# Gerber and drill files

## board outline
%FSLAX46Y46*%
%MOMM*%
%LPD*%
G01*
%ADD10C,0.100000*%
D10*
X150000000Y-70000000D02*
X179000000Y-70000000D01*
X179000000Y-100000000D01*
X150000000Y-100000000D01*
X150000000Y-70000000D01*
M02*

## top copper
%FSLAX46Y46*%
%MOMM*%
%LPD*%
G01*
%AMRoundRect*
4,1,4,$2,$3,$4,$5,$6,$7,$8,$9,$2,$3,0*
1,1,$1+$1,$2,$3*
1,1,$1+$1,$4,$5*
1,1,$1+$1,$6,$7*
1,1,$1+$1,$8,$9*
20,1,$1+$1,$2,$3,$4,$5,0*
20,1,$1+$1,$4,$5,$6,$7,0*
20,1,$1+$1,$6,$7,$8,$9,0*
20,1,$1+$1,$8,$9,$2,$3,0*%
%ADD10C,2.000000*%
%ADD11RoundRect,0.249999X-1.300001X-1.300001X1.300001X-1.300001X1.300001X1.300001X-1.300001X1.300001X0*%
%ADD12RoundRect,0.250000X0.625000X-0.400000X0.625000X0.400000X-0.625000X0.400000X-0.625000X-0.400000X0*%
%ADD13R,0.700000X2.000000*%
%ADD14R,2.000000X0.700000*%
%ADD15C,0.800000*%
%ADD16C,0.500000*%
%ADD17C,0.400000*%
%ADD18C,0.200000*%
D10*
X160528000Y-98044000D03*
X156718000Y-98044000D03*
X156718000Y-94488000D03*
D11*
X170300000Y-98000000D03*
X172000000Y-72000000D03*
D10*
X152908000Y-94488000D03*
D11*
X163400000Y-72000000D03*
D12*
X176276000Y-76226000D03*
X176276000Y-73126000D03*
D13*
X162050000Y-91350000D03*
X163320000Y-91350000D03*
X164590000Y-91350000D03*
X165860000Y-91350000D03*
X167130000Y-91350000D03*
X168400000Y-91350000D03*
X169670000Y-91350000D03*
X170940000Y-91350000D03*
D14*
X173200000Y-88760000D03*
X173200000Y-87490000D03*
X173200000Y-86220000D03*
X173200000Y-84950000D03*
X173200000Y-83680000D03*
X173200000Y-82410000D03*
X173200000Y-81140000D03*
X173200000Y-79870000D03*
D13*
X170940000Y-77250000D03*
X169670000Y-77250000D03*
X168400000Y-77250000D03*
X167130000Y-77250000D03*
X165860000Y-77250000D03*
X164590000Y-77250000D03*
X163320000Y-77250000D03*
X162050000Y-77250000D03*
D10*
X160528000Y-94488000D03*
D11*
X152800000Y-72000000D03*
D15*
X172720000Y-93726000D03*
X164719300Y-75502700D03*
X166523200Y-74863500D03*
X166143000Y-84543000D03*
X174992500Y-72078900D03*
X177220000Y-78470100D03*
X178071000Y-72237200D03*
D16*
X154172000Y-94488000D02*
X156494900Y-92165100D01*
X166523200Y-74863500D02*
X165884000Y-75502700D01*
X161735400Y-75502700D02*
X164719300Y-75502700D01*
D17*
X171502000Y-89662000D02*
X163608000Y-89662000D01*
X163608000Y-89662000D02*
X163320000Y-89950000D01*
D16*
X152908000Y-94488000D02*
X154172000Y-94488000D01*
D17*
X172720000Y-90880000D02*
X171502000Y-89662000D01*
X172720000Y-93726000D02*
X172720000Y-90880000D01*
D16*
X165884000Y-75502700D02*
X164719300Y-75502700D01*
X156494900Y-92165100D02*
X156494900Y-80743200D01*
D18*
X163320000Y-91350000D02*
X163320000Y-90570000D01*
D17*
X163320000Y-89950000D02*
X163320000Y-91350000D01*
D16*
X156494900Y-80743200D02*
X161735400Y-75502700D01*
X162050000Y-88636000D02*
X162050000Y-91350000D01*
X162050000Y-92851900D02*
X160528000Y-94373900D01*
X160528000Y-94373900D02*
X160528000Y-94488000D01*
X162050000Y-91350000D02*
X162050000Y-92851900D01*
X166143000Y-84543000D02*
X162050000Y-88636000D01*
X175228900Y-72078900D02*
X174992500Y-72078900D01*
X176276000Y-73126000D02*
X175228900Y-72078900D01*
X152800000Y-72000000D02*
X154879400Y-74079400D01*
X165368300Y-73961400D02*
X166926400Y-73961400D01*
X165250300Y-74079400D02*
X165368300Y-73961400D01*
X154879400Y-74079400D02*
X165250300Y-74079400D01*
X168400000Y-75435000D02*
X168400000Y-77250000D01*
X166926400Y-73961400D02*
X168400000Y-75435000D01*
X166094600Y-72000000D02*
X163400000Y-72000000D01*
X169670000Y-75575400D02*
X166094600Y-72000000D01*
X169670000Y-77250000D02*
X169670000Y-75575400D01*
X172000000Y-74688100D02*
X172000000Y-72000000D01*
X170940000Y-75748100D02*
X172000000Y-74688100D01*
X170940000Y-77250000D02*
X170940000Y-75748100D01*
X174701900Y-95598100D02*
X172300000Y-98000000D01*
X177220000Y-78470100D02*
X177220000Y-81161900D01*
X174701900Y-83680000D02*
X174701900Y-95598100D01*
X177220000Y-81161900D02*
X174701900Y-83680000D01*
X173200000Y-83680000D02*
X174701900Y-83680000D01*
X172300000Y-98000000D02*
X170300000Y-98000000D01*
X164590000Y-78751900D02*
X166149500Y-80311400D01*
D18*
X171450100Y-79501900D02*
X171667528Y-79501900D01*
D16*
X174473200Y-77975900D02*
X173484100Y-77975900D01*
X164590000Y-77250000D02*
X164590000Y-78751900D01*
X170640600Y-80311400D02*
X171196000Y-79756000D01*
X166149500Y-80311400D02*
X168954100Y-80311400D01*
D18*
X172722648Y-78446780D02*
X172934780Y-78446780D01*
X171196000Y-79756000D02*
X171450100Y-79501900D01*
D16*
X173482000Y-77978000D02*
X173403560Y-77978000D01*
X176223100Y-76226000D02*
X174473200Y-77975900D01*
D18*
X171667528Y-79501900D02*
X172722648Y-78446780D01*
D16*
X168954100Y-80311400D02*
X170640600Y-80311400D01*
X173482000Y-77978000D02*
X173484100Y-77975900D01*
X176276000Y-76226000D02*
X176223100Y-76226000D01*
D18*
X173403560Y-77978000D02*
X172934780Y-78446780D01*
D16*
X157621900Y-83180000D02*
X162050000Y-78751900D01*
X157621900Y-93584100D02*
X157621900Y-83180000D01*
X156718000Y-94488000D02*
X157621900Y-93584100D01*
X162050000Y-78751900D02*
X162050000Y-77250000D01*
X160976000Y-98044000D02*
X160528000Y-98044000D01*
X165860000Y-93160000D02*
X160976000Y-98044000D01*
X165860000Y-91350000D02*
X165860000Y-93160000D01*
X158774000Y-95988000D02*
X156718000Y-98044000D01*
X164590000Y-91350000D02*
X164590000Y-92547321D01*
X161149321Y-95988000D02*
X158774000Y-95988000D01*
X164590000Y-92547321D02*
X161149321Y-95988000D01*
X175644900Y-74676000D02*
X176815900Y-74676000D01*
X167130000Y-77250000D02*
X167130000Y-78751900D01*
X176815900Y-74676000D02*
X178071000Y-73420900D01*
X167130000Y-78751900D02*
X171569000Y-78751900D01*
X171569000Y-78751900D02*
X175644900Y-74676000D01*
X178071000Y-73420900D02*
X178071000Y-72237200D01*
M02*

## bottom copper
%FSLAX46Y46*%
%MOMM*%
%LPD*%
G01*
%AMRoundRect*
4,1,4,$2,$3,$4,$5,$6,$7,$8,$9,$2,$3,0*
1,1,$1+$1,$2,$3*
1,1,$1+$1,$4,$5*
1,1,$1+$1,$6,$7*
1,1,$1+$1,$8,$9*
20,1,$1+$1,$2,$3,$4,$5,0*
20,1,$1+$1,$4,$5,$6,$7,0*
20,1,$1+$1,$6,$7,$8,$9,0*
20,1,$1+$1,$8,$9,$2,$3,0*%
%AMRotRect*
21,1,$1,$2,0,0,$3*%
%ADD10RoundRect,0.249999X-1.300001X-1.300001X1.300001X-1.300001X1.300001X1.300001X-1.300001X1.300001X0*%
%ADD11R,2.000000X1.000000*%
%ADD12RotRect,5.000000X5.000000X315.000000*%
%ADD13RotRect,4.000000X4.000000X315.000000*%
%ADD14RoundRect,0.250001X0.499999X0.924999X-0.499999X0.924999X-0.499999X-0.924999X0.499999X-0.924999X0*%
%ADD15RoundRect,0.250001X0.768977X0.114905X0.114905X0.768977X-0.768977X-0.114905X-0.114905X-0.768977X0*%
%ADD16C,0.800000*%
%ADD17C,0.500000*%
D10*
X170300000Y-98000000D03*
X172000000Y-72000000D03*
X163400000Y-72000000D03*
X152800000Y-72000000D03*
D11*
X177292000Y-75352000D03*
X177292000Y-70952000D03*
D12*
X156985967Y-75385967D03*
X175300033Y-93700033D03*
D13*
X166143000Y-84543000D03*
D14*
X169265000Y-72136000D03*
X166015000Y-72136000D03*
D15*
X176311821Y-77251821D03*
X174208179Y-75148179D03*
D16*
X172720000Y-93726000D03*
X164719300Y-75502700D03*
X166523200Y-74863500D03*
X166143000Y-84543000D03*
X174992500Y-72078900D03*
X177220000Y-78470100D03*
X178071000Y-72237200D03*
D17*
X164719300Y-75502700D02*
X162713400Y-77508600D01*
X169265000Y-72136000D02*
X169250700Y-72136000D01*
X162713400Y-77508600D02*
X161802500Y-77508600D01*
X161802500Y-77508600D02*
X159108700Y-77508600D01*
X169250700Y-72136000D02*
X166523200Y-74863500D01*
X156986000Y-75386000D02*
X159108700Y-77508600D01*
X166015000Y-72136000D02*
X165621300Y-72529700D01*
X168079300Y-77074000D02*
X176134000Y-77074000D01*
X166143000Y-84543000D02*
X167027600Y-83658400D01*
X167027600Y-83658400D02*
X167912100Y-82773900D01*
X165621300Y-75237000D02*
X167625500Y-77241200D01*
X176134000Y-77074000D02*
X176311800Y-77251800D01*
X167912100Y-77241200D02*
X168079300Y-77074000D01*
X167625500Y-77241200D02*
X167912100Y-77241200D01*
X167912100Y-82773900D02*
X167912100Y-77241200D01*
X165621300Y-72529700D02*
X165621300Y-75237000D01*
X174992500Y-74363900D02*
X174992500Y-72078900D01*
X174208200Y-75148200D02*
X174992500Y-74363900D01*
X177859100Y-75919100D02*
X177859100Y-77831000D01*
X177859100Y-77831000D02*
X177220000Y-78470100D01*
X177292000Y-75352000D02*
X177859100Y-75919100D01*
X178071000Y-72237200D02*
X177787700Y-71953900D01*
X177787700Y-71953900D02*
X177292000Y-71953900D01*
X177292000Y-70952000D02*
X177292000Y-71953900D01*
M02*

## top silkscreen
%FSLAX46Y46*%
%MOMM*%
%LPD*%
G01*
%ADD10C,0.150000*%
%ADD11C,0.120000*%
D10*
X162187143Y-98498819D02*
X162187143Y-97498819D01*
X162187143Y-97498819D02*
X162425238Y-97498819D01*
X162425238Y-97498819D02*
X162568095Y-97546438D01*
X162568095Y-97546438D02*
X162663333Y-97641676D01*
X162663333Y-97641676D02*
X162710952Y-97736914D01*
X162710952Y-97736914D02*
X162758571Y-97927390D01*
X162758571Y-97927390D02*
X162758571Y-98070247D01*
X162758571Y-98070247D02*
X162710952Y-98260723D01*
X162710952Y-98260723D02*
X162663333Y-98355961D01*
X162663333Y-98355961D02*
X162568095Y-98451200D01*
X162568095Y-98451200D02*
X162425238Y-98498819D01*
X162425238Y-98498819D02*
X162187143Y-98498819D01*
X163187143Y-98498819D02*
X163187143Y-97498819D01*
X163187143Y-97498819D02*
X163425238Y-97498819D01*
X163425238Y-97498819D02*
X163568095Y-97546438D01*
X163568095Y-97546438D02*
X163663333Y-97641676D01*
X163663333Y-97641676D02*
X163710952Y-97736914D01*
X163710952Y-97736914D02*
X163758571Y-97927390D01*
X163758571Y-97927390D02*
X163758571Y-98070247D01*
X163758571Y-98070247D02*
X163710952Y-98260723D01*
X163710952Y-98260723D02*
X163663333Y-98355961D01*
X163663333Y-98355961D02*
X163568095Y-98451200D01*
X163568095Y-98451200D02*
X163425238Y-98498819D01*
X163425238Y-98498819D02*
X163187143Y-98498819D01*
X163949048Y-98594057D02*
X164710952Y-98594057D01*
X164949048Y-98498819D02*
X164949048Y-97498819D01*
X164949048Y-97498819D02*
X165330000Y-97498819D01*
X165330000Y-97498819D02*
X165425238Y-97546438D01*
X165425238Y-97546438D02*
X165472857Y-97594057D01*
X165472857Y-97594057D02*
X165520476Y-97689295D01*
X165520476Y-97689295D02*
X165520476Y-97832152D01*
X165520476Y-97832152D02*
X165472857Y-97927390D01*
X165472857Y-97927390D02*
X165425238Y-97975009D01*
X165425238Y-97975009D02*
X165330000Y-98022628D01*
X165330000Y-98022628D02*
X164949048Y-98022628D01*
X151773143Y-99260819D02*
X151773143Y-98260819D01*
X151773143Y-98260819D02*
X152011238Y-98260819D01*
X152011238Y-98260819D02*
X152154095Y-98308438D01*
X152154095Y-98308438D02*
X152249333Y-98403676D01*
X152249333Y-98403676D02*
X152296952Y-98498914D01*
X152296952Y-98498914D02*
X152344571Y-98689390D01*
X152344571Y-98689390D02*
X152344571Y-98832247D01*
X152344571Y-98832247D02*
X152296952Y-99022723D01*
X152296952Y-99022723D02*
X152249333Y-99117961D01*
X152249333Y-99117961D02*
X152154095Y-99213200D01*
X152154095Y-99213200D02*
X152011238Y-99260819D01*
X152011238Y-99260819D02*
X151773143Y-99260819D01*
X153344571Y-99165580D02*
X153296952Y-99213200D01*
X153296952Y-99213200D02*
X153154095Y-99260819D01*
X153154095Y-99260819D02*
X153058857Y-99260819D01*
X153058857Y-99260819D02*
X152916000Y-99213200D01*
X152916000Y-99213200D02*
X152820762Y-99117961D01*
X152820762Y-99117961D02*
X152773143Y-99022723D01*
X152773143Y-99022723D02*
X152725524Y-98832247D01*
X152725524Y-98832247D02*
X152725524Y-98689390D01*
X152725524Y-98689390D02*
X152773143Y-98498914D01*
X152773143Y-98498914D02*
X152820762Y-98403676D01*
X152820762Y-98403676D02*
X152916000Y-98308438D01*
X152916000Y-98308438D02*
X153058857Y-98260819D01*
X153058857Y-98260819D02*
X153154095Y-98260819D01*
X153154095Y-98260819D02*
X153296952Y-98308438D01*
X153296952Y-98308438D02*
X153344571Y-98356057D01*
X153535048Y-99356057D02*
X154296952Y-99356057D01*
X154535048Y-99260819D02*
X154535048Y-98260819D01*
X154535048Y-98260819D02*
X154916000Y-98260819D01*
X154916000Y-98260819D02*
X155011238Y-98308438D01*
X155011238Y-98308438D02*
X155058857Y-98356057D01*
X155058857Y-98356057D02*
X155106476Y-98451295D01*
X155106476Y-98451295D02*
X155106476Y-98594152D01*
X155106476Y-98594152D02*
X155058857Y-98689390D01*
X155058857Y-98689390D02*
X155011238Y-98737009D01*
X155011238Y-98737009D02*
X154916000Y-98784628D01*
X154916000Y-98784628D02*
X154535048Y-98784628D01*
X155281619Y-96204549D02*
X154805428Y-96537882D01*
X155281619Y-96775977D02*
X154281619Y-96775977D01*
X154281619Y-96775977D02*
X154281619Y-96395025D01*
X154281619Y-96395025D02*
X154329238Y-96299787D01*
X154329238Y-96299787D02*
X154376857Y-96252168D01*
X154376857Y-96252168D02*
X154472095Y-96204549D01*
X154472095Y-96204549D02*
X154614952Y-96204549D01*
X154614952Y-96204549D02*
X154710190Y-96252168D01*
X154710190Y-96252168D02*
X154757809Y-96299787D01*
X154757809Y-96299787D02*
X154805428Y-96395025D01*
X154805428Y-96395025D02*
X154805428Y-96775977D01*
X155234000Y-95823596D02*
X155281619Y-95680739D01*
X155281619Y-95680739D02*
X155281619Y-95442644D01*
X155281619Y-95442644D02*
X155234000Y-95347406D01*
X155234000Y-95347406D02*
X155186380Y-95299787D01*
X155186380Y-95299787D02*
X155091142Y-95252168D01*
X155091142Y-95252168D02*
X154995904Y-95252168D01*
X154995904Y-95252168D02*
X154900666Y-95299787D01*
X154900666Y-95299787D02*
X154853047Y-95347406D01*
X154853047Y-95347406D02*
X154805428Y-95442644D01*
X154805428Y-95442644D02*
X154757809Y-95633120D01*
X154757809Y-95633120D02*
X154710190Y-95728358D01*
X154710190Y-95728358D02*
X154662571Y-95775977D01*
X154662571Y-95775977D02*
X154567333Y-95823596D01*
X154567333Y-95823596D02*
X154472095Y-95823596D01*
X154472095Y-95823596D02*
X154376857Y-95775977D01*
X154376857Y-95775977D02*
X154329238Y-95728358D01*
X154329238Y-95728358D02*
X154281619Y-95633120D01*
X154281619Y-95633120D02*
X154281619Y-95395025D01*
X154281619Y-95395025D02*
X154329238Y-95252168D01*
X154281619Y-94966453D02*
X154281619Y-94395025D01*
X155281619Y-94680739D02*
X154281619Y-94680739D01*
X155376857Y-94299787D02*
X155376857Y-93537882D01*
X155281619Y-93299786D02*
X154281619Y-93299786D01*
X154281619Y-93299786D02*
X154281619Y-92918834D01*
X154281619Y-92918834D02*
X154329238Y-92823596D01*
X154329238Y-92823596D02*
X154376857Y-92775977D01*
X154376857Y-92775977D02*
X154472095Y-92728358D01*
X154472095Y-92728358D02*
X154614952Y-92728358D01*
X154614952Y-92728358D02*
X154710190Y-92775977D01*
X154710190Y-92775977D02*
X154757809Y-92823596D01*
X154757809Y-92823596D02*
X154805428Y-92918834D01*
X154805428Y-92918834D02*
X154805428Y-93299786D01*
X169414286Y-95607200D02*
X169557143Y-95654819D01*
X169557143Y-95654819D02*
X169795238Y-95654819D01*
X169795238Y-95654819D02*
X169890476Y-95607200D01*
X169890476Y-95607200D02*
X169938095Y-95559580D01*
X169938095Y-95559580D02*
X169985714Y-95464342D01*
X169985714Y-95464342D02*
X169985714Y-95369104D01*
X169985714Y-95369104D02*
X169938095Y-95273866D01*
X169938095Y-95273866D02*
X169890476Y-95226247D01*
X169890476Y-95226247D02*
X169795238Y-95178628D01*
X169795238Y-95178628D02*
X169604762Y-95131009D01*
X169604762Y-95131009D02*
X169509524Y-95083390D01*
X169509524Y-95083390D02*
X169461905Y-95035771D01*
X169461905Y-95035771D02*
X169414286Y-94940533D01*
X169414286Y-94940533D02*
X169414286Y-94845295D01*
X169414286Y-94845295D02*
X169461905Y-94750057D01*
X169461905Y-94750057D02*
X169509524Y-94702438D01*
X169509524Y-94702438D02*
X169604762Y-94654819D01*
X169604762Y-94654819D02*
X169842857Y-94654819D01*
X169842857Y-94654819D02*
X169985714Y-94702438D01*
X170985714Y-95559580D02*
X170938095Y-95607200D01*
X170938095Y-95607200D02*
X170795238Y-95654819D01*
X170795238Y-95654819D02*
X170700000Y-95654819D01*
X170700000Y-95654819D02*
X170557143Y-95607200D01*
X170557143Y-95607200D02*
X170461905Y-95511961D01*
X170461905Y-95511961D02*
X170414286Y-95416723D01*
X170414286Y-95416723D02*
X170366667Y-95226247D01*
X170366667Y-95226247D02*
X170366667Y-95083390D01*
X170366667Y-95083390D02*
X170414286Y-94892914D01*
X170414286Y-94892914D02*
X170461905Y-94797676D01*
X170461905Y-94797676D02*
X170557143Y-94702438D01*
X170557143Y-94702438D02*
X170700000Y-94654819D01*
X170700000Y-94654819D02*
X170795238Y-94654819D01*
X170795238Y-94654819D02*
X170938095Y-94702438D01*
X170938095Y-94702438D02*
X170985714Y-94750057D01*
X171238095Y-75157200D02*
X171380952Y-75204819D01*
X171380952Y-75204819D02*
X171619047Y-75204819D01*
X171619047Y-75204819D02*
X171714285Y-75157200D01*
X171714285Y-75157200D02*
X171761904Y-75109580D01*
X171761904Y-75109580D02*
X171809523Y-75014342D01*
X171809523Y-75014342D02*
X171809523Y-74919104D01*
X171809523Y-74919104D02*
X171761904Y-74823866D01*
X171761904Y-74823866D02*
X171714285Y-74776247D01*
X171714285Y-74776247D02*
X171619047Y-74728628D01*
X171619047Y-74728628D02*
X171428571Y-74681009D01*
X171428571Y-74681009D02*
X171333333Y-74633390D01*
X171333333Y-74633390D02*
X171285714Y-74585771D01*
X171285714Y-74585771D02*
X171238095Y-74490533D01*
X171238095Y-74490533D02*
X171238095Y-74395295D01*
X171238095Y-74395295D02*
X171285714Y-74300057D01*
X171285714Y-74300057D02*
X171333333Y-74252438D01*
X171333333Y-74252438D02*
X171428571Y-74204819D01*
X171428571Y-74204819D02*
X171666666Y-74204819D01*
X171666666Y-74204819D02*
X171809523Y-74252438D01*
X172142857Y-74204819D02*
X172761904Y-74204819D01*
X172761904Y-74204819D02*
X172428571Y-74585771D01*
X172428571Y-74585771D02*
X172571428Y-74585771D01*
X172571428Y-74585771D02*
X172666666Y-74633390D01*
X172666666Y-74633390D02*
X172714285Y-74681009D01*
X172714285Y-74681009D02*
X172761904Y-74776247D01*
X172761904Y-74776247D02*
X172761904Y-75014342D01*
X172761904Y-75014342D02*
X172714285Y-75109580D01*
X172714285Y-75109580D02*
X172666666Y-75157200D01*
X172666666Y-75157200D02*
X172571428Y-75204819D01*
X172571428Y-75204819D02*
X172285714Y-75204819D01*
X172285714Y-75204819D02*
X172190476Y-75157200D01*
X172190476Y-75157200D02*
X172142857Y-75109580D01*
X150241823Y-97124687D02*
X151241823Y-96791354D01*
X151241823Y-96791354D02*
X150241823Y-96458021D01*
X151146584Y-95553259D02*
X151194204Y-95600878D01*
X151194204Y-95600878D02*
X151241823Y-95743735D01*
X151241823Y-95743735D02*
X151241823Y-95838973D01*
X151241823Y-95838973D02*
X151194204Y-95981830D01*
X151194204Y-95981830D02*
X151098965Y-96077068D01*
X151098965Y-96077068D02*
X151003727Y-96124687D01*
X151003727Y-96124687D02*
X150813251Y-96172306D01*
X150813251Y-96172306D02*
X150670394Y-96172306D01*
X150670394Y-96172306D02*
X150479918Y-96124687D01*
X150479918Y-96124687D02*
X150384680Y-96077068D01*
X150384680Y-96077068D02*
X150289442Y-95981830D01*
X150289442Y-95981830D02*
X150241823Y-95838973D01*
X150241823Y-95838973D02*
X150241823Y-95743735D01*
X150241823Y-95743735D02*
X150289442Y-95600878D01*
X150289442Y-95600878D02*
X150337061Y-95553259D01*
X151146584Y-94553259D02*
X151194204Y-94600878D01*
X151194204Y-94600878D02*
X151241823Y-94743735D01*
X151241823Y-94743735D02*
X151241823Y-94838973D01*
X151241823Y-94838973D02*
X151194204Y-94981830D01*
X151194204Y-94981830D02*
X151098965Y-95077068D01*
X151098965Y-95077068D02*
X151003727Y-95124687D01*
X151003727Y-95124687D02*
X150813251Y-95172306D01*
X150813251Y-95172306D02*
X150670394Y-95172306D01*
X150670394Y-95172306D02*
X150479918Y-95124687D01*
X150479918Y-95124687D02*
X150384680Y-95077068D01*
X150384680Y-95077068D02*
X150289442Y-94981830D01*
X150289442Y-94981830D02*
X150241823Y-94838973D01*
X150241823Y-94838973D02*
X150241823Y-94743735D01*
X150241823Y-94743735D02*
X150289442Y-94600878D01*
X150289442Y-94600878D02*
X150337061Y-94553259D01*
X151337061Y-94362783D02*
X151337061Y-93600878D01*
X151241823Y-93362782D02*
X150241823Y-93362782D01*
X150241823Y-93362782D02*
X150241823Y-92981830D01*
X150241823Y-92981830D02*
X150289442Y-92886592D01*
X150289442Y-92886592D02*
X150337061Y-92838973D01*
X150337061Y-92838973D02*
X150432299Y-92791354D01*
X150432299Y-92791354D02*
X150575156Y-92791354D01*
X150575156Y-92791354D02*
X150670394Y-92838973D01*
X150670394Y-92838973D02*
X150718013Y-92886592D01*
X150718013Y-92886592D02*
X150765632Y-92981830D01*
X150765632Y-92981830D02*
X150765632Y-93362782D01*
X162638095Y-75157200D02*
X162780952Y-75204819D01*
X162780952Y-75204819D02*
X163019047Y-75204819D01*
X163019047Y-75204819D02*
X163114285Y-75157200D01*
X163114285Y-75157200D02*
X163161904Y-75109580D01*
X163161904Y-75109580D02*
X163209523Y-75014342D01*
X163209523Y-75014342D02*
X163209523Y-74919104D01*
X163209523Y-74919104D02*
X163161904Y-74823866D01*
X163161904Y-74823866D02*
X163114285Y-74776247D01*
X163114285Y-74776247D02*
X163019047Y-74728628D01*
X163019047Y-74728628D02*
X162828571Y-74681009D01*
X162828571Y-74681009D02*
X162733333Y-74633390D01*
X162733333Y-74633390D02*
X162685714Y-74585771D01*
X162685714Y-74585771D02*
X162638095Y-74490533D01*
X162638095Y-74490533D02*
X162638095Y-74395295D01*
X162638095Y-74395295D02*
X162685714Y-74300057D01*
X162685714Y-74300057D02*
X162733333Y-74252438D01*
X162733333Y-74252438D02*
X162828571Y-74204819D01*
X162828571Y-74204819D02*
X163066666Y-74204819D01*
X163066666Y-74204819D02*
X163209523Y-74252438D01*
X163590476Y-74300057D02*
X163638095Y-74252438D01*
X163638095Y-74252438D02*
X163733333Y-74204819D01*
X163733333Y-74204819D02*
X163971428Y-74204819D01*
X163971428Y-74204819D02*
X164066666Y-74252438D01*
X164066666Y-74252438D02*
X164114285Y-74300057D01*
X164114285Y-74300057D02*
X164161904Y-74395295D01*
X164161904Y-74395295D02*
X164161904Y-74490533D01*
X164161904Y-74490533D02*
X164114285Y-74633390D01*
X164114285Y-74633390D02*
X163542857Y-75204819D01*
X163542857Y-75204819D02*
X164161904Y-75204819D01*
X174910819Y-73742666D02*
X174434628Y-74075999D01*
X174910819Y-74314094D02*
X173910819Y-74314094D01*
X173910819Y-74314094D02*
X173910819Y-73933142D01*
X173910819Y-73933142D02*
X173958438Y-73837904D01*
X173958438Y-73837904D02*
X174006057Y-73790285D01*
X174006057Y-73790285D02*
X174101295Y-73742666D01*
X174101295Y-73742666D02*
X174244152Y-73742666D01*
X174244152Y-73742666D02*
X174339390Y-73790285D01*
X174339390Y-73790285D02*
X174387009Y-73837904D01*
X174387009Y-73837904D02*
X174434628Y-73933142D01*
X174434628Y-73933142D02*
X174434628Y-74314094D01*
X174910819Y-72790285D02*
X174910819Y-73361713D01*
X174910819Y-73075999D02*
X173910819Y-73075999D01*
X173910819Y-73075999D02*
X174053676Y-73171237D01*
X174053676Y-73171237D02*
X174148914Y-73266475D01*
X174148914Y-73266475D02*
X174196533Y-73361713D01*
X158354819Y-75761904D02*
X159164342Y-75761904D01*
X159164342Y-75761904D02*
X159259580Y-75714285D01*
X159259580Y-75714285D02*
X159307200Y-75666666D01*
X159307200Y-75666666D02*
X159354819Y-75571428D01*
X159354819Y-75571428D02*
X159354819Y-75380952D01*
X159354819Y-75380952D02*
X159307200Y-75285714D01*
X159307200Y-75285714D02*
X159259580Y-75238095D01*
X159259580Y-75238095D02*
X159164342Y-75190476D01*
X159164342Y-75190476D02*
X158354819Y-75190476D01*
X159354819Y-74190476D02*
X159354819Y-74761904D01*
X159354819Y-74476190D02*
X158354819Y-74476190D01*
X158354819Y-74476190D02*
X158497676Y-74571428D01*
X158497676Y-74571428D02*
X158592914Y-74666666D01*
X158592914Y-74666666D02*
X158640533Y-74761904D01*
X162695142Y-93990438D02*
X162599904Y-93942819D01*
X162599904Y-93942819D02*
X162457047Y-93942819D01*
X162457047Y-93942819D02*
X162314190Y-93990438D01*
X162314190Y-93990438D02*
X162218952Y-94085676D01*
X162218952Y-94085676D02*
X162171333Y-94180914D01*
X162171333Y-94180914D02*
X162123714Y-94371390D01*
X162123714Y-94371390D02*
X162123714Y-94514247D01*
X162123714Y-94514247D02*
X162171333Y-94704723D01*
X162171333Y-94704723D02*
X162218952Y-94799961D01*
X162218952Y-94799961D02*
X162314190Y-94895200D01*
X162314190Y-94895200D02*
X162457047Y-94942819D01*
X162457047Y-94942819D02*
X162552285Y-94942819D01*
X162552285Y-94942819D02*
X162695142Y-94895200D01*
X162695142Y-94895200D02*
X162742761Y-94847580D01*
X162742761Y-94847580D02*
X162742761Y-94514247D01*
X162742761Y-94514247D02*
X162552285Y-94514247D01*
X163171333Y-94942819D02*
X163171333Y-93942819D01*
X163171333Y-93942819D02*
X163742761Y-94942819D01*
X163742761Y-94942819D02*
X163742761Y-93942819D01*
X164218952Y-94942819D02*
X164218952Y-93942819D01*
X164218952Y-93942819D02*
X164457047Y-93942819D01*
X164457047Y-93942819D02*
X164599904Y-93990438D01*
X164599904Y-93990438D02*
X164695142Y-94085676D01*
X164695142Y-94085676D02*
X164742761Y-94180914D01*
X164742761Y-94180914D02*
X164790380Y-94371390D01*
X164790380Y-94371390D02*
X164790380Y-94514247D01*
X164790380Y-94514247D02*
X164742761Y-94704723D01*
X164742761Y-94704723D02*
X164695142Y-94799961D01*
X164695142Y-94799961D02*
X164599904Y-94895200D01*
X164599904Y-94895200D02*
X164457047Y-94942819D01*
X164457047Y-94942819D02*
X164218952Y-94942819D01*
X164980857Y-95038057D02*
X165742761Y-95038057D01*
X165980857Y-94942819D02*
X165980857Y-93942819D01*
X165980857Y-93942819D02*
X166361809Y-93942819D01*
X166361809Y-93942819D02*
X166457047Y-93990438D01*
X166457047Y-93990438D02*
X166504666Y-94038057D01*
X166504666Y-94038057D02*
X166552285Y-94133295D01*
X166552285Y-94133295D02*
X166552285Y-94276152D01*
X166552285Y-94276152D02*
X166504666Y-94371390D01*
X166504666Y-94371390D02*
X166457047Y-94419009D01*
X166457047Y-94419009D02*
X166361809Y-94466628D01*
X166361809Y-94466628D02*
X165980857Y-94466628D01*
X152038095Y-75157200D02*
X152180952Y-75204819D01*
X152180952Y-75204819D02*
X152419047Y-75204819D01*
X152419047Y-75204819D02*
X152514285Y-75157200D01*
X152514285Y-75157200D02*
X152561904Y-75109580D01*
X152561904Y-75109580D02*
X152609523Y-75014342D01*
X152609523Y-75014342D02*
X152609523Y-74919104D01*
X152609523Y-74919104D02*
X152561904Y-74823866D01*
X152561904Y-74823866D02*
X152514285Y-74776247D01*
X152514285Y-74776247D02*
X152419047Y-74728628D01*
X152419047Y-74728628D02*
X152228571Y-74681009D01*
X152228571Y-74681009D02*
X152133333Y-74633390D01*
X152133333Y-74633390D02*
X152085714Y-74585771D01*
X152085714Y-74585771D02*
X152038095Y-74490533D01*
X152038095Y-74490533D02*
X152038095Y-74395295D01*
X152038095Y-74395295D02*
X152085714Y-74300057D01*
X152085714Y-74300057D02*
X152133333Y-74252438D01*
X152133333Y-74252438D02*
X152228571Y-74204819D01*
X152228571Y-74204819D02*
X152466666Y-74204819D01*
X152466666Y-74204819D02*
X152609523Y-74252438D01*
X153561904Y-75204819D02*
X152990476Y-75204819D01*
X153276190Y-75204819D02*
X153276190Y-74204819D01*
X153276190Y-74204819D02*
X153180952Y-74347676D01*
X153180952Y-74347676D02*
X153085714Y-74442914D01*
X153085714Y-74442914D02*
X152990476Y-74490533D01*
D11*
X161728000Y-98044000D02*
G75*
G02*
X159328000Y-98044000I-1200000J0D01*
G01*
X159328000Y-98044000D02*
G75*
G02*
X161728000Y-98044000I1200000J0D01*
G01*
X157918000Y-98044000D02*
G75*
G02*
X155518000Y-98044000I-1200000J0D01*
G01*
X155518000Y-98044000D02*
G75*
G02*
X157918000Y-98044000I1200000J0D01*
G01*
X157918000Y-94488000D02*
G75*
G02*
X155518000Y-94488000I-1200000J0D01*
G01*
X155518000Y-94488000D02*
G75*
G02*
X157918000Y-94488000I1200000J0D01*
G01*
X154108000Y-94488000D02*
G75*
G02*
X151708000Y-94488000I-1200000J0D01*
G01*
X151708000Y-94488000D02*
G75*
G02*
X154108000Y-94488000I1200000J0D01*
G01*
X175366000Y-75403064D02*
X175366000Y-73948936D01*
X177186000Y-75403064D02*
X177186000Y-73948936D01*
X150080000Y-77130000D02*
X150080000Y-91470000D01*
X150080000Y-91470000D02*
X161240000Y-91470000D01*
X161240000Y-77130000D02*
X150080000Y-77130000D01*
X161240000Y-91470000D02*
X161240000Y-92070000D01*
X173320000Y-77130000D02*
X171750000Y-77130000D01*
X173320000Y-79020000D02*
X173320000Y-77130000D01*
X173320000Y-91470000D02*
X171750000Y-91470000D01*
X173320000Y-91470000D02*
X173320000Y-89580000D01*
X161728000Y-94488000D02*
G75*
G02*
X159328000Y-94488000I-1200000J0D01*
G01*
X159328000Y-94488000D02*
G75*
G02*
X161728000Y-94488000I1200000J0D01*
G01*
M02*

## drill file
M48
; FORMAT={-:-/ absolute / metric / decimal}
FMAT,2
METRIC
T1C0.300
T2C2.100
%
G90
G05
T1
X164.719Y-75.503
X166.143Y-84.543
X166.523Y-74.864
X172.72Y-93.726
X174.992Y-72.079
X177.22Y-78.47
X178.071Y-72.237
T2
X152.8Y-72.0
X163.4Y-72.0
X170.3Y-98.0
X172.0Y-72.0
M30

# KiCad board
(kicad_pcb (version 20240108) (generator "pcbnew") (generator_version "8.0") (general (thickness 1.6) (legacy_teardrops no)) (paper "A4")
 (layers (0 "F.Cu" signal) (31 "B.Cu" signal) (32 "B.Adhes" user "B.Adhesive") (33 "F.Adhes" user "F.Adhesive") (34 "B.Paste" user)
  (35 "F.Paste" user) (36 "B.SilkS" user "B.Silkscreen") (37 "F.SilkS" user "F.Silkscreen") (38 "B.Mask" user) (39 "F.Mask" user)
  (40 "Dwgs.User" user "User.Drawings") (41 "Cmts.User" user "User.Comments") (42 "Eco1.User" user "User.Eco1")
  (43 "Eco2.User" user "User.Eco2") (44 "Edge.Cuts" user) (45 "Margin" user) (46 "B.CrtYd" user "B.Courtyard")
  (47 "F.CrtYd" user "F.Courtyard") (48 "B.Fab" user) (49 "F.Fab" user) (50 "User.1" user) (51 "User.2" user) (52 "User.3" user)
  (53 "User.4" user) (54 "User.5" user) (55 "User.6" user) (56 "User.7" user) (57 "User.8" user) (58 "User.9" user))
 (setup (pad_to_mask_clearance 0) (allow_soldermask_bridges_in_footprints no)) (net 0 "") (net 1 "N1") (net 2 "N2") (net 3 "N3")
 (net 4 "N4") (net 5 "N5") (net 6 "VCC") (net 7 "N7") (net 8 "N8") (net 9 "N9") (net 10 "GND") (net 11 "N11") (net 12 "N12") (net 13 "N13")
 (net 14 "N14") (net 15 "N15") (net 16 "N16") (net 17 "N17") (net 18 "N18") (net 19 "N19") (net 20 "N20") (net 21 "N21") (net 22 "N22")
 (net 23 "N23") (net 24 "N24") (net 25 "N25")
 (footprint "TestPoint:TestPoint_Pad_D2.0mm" (layer "F.Cu") (at 160.528 98.044 -90)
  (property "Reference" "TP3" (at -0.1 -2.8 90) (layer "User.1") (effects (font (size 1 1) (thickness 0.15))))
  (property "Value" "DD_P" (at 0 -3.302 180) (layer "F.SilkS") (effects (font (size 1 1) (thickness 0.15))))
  (fp_circle (center 0 0) (end 0 1.2) (stroke (width 0.12) (type solid)) (fill none) (layer "F.SilkS"))
  (pad "1" smd circle (at 0 0 270) (size 2 2) (layers "F.Cu" "F.Mask") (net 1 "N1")))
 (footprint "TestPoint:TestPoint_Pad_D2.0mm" (layer "F.Cu") (at 156.718 98.044 -90)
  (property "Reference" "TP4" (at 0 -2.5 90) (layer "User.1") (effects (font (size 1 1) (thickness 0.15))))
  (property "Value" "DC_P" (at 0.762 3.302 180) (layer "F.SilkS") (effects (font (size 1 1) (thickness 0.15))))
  (fp_circle (center 0 0) (end 0 1.2) (stroke (width 0.12) (type solid)) (fill none) (layer "F.SilkS"))
  (pad "1" smd circle (at 0 0 270) (size 2 2) (layers "F.Cu" "F.Mask") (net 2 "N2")))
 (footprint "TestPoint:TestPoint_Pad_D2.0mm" (layer "F.Cu") (at 156.718 94.488 -90)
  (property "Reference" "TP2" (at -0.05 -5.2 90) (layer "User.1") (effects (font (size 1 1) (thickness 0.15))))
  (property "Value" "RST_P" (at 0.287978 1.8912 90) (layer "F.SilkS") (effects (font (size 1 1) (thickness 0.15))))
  (fp_circle (center 0 0) (end 0 1.2) (stroke (width 0.12) (type solid)) (fill none) (layer "F.SilkS"))
  (pad "1" smd circle (at 0 0 270) (size 2 2) (layers "F.Cu" "F.Mask") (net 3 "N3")))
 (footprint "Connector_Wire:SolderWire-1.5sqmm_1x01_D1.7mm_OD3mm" (layer "F.Cu") (at 170.3 98)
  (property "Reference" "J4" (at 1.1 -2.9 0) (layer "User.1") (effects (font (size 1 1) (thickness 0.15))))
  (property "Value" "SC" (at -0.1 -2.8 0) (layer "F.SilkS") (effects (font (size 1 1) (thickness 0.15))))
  (pad "1" thru_hole roundrect (at 0 0) (size 3.1 3.1) (drill 2.1) (layers "*.Cu" "*.Mask") (remove_unused_layers no)
   (roundrect_rratio 0.08064483871) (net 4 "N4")))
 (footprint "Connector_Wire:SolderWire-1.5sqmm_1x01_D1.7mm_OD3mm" (layer "F.Cu") (at 172 72)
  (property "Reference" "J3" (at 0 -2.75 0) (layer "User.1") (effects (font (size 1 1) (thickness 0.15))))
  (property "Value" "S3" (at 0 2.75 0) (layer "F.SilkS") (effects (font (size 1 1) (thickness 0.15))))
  (pad "1" thru_hole roundrect (at 0 0) (size 3.1 3.1) (drill 2.1) (layers "*.Cu" "*.Mask") (remove_unused_layers no)
   (roundrect_rratio 0.08064483871) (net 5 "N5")))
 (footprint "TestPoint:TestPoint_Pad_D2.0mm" (layer "F.Cu") (at 152.908 94.488 -90)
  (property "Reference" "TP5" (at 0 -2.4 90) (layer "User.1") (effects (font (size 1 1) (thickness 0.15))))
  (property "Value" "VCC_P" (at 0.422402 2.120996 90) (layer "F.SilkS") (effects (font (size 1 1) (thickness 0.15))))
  (fp_circle (center 0 0) (end 0 1.2) (stroke (width 0.12) (type solid)) (fill none) (layer "F.SilkS"))
  (pad "1" smd circle (at 0 0 270) (size 2 2) (layers "F.Cu" "F.Mask") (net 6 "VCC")))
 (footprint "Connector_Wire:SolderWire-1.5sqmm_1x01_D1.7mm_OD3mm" (layer "F.Cu") (at 163.4 72)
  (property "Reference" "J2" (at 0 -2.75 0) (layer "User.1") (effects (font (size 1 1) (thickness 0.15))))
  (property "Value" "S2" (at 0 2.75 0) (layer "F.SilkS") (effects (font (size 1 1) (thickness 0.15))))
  (pad "1" thru_hole roundrect (at 0 0) (size 3.1 3.1) (drill 2.1) (layers "*.Cu" "*.Mask") (remove_unused_layers no)
   (roundrect_rratio 0.08064483871) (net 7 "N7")))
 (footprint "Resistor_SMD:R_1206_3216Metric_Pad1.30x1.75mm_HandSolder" (layer "F.Cu") (at 176.276 74.676 90)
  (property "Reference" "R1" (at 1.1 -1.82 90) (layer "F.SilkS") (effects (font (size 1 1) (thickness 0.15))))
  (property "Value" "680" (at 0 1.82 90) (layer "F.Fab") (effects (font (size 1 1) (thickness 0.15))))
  (fp_line (start -0.727064 -0.91) (end 0.727064 -0.91) (stroke (width 0.12) (type solid)) (layer "F.SilkS"))
  (fp_line (start -0.727064 0.91) (end 0.727064 0.91) (stroke (width 0.12) (type solid)) (layer "F.SilkS"))
  (pad "1" smd roundrect (at -1.55 0 90) (size 1.3 1.75) (layers "F.Cu" "F.Paste" "F.Mask") (roundrect_rratio 0.1923076923) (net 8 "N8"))
  (pad "2" smd roundrect (at 1.55 0 90) (size 1.3 1.75) (layers "F.Cu" "F.Paste" "F.Mask") (roundrect_rratio 0.1923076923) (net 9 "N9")))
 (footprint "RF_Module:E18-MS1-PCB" (layer "F.Cu") (at 161.7 84.3 90)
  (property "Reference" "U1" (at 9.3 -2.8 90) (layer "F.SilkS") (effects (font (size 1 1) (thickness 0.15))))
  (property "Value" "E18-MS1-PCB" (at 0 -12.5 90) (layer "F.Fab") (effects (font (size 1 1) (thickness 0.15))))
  (fp_line (start 7.17 -11.62) (end -7.17 -11.62) (stroke (width 0.12) (type solid)) (layer "F.SilkS"))
  (fp_line (start -7.17 -11.62) (end -7.17 -0.46) (stroke (width 0.12) (type solid)) (layer "F.SilkS"))
  (fp_line (start 7.17 -0.46) (end 7.17 -11.62) (stroke (width 0.12) (type solid)) (layer "F.SilkS"))
  (fp_line (start -7.17 -0.46) (end -7.77 -0.46) (stroke (width 0.12) (type solid)) (layer "F.SilkS"))
  (fp_line (start 7.17 11.62) (end 7.17 10.05) (stroke (width 0.12) (type solid)) (layer "F.SilkS"))
  (fp_line (start 5.28 11.62) (end 7.17 11.62) (stroke (width 0.12) (type solid)) (layer "F.SilkS"))
  (fp_line (start -7.17 11.62) (end -7.17 10.05) (stroke (width 0.12) (type solid)) (layer "F.SilkS"))
  (fp_line (start -7.17 11.62) (end -5.28 11.62) (stroke (width 0.12) (type solid)) (layer "F.SilkS"))
  (pad "1" smd rect (at -7.05 0.35) (size 0.7 2) (layers "F.Cu" "F.Paste" "F.Mask") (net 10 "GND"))
  (pad "2" smd rect (at -7.05 1.62) (size 0.7 2) (layers "F.Cu" "F.Paste" "F.Mask") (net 6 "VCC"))
  (pad "3" smd rect (at -7.05 2.89) (size 0.7 2) (layers "F.Cu" "F.Paste" "F.Mask") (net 2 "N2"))
  (pad "4" smd rect (at -7.05 4.16) (size 0.7 2) (layers "F.Cu" "F.Paste" "F.Mask") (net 1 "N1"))
  (pad "5" smd rect (at -7.05 5.43) (size 0.7 2) (layers "F.Cu" "F.Paste" "F.Mask") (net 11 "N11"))
  (pad "6" smd rect (at -7.05 6.7) (size 0.7 2) (layers "F.Cu" "F.Paste" "F.Mask") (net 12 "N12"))
  (pad "7" smd rect (at -7.05 7.97) (size 0.7 2) (layers "F.Cu" "F.Paste" "F.Mask") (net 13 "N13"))
  (pad "8" smd rect (at -7.05 9.24) (size 0.7 2) (layers "F.Cu" "F.Paste" "F.Mask") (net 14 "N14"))
  (pad "9" smd rect (at -4.46 11.5 270) (size 0.7 2) (layers "F.Cu" "F.Paste" "F.Mask") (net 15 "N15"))
  (pad "10" smd rect (at -3.19 11.5 270) (size 0.7 2) (layers "F.Cu" "F.Paste" "F.Mask") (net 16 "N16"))
  (pad "11" smd rect (at -1.92 11.5 270) (size 0.7 2) (layers "F.Cu" "F.Paste" "F.Mask") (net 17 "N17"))
  (pad "12" smd rect (at -0.65 11.5 270) (size 0.7 2) (layers "F.Cu" "F.Paste" "F.Mask") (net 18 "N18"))
  (pad "13" smd rect (at 0.62 11.5 270) (size 0.7 2) (layers "F.Cu" "F.Paste" "F.Mask") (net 4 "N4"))
  (pad "14" smd rect (at 1.89 11.5 270) (size 0.7 2) (layers "F.Cu" "F.Paste" "F.Mask") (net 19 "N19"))
  (pad "15" smd rect (at 3.16 11.5 270) (size 0.7 2) (layers "F.Cu" "F.Paste" "F.Mask") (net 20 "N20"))
  (pad "16" smd rect (at 4.43 11.5 270) (size 0.7 2) (layers "F.Cu" "F.Paste" "F.Mask") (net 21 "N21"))
  (pad "17" smd rect (at 7.05 9.24 180) (size 0.7 2) (layers "F.Cu" "F.Paste" "F.Mask") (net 5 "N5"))
  (pad "18" smd rect (at 7.05 7.97 180) (size 0.7 2) (layers "F.Cu" "F.Paste" "F.Mask") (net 7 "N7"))
  (pad "19" smd rect (at 7.05 6.7 180) (size 0.7 2) (layers "F.Cu" "F.Paste" "F.Mask") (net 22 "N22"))
  (pad "20" smd rect (at 7.05 5.43 180) (size 0.7 2) (layers "F.Cu" "F.Paste" "F.Mask") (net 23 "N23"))
  (pad "21" smd rect (at 7.05 4.16 180) (size 0.7 2) (layers "F.Cu" "F.Paste" "F.Mask") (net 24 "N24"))
  (pad "22" smd rect (at 7.05 2.89 180) (size 0.7 2) (layers "F.Cu" "F.Paste" "F.Mask") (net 8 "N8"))
  (pad "23" smd rect (at 7.05 1.62 180) (size 0.7 2) (layers "F.Cu" "F.Paste" "F.Mask") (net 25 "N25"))
  (pad "24" smd rect (at 7.05 0.35 180) (size 0.7 2) (layers "F.Cu" "F.Paste" "F.Mask") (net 3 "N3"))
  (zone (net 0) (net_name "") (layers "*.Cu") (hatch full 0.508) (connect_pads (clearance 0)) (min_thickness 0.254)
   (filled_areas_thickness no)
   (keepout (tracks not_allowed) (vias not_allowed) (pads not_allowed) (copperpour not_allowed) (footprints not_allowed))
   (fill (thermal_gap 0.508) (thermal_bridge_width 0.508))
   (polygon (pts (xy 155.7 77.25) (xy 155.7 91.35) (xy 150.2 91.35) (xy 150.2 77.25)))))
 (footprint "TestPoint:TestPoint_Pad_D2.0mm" (layer "F.Cu") (at 160.528 94.488 -90)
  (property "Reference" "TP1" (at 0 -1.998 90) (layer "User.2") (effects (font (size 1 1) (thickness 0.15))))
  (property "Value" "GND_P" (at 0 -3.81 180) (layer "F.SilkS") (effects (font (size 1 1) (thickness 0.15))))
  (fp_circle (center 0 0) (end 0 1.2) (stroke (width 0.12) (type solid)) (fill none) (layer "F.SilkS"))
  (pad "1" smd circle (at 0 0 270) (size 2 2) (layers "F.Cu" "F.Mask") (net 10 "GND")))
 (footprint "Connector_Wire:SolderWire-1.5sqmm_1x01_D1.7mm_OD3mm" (layer "F.Cu") (at 152.8 72)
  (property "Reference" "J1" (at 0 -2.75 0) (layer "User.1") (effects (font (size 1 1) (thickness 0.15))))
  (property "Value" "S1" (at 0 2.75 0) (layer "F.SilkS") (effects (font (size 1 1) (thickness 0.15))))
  (pad "1" thru_hole roundrect (at 0 0) (size 3.1 3.1) (drill 2.1) (layers "*.Cu" "*.Mask") (remove_unused_layers no)
   (roundrect_rratio 0.08064483871) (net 22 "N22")))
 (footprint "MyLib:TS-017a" (layer "B.Cu") (at 177.292 73.152 90)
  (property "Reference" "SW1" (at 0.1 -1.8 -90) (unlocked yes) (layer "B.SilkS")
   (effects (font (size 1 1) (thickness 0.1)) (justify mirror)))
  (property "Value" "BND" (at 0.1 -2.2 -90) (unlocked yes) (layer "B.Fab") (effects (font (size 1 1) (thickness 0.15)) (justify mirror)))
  (pad "1" smd rect (at -2.2 0) (size 2 1) (layers "B.Cu" "B.Paste" "B.Mask") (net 4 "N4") (thermal_bridge_angle 45))
  (pad "2" smd rect (at 2.2 0) (size 2 1) (layers "B.Cu" "B.Paste" "B.Mask") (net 23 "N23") (thermal_bridge_angle 45)))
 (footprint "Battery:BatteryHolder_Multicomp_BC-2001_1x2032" (layer "B.Cu") (at 166.143 84.543 -45)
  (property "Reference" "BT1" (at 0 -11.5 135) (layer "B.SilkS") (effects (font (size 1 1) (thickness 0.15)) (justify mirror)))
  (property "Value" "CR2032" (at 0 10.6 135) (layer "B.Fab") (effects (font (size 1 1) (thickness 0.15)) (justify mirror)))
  (pad "1" smd rect (at -12.95 0 315) (size 5 5) (layers "B.Cu" "B.Paste" "B.Mask") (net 6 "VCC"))
  (pad "1" smd rect (at 12.95 0 315) (size 5 5) (layers "B.Cu" "B.Paste" "B.Mask") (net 6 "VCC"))
  (pad "2" smd rect (at 0 0 315) (size 4 4) (layers "B.Cu" "B.Paste" "B.Mask") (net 10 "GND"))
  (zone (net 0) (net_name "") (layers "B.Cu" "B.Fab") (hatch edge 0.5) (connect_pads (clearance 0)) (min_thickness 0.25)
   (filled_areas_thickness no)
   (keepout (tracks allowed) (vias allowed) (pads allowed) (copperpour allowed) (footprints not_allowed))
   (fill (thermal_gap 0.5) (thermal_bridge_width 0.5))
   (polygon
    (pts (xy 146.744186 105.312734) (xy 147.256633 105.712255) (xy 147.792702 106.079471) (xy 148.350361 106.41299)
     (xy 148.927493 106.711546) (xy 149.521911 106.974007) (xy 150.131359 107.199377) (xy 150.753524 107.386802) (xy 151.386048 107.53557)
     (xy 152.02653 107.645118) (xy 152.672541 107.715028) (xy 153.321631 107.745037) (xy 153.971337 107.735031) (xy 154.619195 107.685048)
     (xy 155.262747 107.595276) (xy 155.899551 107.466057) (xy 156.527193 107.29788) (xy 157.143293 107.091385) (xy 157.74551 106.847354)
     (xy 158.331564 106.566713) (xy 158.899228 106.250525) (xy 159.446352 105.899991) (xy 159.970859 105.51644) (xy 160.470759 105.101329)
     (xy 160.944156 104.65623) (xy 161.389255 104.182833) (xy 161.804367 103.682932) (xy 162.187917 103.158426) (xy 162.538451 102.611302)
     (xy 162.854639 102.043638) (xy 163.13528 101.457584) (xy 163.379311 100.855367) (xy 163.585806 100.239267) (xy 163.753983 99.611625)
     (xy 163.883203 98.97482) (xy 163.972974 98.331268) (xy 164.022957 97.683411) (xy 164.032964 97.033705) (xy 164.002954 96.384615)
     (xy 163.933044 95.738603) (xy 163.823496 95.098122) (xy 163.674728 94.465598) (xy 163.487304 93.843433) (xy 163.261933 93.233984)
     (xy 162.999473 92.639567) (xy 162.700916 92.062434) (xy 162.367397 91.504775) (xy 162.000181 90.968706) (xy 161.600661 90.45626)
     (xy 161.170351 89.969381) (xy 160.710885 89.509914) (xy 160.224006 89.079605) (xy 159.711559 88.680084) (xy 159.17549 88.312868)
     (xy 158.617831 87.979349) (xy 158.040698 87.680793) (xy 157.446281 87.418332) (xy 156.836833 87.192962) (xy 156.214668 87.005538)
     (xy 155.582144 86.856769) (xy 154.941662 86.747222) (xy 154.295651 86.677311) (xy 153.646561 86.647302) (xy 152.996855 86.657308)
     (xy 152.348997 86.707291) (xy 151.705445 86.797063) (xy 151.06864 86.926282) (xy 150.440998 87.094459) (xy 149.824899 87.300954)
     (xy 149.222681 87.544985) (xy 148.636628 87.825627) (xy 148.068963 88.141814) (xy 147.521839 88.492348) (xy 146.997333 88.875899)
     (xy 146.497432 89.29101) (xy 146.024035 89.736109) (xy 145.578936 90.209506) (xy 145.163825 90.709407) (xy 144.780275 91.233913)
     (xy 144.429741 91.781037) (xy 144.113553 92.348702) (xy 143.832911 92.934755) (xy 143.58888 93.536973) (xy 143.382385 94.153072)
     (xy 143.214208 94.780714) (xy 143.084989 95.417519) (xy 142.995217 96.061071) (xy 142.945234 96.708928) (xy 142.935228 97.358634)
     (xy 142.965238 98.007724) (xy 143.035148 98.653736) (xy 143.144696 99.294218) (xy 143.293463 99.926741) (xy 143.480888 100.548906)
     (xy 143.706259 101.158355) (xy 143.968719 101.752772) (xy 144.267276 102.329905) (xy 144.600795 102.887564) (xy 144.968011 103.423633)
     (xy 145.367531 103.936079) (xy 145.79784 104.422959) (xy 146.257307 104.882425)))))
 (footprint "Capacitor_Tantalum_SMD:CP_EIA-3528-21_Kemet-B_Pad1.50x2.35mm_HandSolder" (layer "B.Cu") (at 167.64 72.136 180)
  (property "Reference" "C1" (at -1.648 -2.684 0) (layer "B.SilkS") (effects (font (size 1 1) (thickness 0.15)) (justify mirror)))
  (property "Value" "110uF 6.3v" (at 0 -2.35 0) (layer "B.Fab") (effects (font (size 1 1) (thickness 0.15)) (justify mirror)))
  (pad "1" smd roundrect (at -1.625 0 180) (size 1.5 2.35) (layers "B.Cu" "B.Paste" "B.Mask") (roundrect_rratio 0.1666673333) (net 6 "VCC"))
  (pad "2" smd roundrect (at 1.625 0 180) (size 1.5 2.35) (layers "B.Cu" "B.Paste" "B.Mask") (roundrect_rratio 0.1666673333) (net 10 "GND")))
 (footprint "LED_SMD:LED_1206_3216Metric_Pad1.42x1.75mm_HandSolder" (layer "B.Cu") (at 175.26 76.2 135)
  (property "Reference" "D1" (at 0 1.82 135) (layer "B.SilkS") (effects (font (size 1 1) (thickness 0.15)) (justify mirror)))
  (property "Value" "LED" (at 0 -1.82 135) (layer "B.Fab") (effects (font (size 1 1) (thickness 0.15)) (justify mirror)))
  (pad "1" smd roundrect (at -1.4875 0 135) (size 1.425 1.75) (layers "B.Cu" "B.Paste" "B.Mask") (roundrect_rratio 0.1754392982)
   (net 10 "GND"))
  (pad "2" smd roundrect (at 1.4875 0 135) (size 1.425 1.75) (layers "B.Cu" "B.Paste" "B.Mask") (roundrect_rratio 0.1754392982) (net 9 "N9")))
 (gr_rect (start 150 70) (end 179 100) (stroke (width 0.1) (type default)) (fill none) (layer "Edge.Cuts"))
 (segment (start 154.172 94.488) (end 156.4949 92.1651) (width 0.5) (layer "F.Cu") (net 6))
 (segment (start 166.5232 74.8635) (end 165.884 75.5027) (width 0.5) (layer "F.Cu") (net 6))
 (segment (start 161.7354 75.5027) (end 164.7193 75.5027) (width 0.5) (layer "F.Cu") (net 6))
 (segment (start 171.502 89.662) (end 163.608 89.662) (width 0.4) (layer "F.Cu") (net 6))
 (segment (start 163.608 89.662) (end 163.32 89.95) (width 0.4) (layer "F.Cu") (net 6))
 (segment (start 152.908 94.488) (end 154.172 94.488) (width 0.5) (layer "F.Cu") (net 6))
 (segment (start 172.72 90.88) (end 171.502 89.662) (width 0.4) (layer "F.Cu") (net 6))
 (segment (start 172.72 93.726) (end 172.72 90.88) (width 0.4) (layer "F.Cu") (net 6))
 (segment (start 165.884 75.5027) (end 164.7193 75.5027) (width 0.5) (layer "F.Cu") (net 6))
 (segment (start 156.4949 92.1651) (end 156.4949 80.7432) (width 0.5) (layer "F.Cu") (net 6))
 (segment (start 163.32 91.35) (end 163.32 90.57) (width 0.2) (layer "F.Cu") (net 6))
 (segment (start 163.32 89.95) (end 163.32 91.35) (width 0.4) (layer "F.Cu") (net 6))
 (segment (start 156.4949 80.7432) (end 161.7354 75.5027) (width 0.5) (layer "F.Cu") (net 6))
 (via (at 172.72 93.726) (size 0.8) (drill 0.3) (layers "F.Cu" "B.Cu") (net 6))
 (via (at 164.7193 75.5027) (size 0.8) (drill 0.3) (layers "F.Cu" "B.Cu") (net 6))
 (via (at 166.5232 74.8635) (size 0.8) (drill 0.3) (layers "F.Cu" "B.Cu") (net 6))
 (segment (start 164.7193 75.5027) (end 162.7134 77.5086) (width 0.5) (layer "B.Cu") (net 6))
 (segment (start 169.265 72.136) (end 169.2507 72.136) (width 0.5) (layer "B.Cu") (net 6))
 (segment (start 162.7134 77.5086) (end 161.8025 77.5086) (width 0.5) (layer "B.Cu") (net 6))
 (segment (start 161.8025 77.5086) (end 159.1087 77.5086) (width 0.5) (layer "B.Cu") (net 6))
 (segment (start 169.2507 72.136) (end 166.5232 74.8635) (width 0.5) (layer "B.Cu") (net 6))
 (segment (start 156.986 75.386) (end 159.1087 77.5086) (width 0.5) (layer "B.Cu") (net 6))
 (segment (start 162.05 88.636) (end 162.05 91.35) (width 0.5) (layer "F.Cu") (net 10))
 (segment (start 162.05 92.8519) (end 160.528 94.3739) (width 0.5) (layer "F.Cu") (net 10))
 (segment (start 160.528 94.3739) (end 160.528 94.488) (width 0.5) (layer "F.Cu") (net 10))
 (segment (start 162.05 91.35) (end 162.05 92.8519) (width 0.5) (layer "F.Cu") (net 10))
 (segment (start 166.143 84.543) (end 162.05 88.636) (width 0.5) (layer "F.Cu") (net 10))
 (via (at 166.143 84.543) (size 0.8) (drill 0.3) (layers "F.Cu" "B.Cu") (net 10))
 (segment (start 166.015 72.136) (end 165.6213 72.5297) (width 0.5) (layer "B.Cu") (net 10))
 (segment (start 168.0793 77.074) (end 176.134 77.074) (width 0.5) (layer "B.Cu") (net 10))
 (segment (start 166.143 84.543) (end 167.0276 83.6584) (width 0.5) (layer "B.Cu") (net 10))
 (segment (start 167.0276 83.6584) (end 167.9121 82.7739) (width 0.5) (layer "B.Cu") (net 10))
 (segment (start 165.6213 75.237) (end 167.6255 77.2412) (width 0.5) (layer "B.Cu") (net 10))
 (segment (start 176.134 77.074) (end 176.3118 77.2518) (width 0.5) (layer "B.Cu") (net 10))
 (segment (start 167.9121 77.2412) (end 168.0793 77.074) (width 0.5) (layer "B.Cu") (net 10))
 (segment (start 167.6255 77.2412) (end 167.9121 77.2412) (width 0.5) (layer "B.Cu") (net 10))
 (segment (start 167.9121 82.7739) (end 167.9121 77.2412) (width 0.5) (layer "B.Cu") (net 10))
 (segment (start 165.6213 72.5297) (end 165.6213 75.237) (width 0.5) (layer "B.Cu") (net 10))
 (segment (start 175.2289 72.0789) (end 174.9925 72.0789) (width 0.5) (layer "F.Cu") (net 9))
 (segment (start 176.276 73.126) (end 175.2289 72.0789) (width 0.5) (layer "F.Cu") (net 9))
 (via (at 174.9925 72.0789) (size 0.8) (drill 0.3) (layers "F.Cu" "B.Cu") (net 9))
 (segment (start 174.9925 74.3639) (end 174.9925 72.0789) (width 0.5) (layer "B.Cu") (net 9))
 (segment (start 174.2082 75.1482) (end 174.9925 74.3639) (width 0.5) (layer "B.Cu") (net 9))
 (segment (start 152.8 72) (end 154.8794 74.0794) (width 0.5) (layer "F.Cu") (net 22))
 (segment (start 165.3683 73.9614) (end 166.9264 73.9614) (width 0.5) (layer "F.Cu") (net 22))
 (segment (start 165.2503 74.0794) (end 165.3683 73.9614) (width 0.5) (layer "F.Cu") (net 22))
 (segment (start 154.8794 74.0794) (end 165.2503 74.0794) (width 0.5) (layer "F.Cu") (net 22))
 (segment (start 168.4 75.435) (end 168.4 77.25) (width 0.5) (layer "F.Cu") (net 22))
 (segment (start 166.9264 73.9614) (end 168.4 75.435) (width 0.5) (layer "F.Cu") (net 22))
 (segment (start 166.0946 72) (end 163.4 72) (width 0.5) (layer "F.Cu") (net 7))
 (segment (start 169.67 75.5754) (end 166.0946 72) (width 0.5) (layer "F.Cu") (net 7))
 (segment (start 169.67 77.25) (end 169.67 75.5754) (width 0.5) (layer "F.Cu") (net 7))
 (segment (start 172 74.6881) (end 172 72) (width 0.5) (layer "F.Cu") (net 5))
 (segment (start 170.94 75.7481) (end 172 74.6881) (width 0.5) (layer "F.Cu") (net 5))
 (segment (start 170.94 77.25) (end 170.94 75.7481) (width 0.5) (layer "F.Cu") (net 5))
 (segment (start 174.7019 95.5981) (end 172.3 98) (width 0.5) (layer "F.Cu") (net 4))
 (segment (start 177.22 78.4701) (end 177.22 81.1619) (width 0.5) (layer "F.Cu") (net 4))
 (segment (start 174.7019 83.68) (end 174.7019 95.5981) (width 0.5) (layer "F.Cu") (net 4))
 (segment (start 177.22 81.1619) (end 174.7019 83.68) (width 0.5) (layer "F.Cu") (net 4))
 (segment (start 173.2 83.68) (end 174.7019 83.68) (width 0.5) (layer "F.Cu") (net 4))
 (segment (start 172.3 98) (end 170.3 98) (width 0.5) (layer "F.Cu") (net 4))
 (via (at 177.22 78.4701) (size 0.8) (drill 0.3) (layers "F.Cu" "B.Cu") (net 4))
 (segment (start 177.8591 75.9191) (end 177.8591 77.831) (width 0.5) (layer "B.Cu") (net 4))
 (segment (start 177.8591 77.831) (end 177.22 78.4701) (width 0.5) (layer "B.Cu") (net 4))
 (segment (start 177.292 75.352) (end 177.8591 75.9191) (width 0.5) (layer "B.Cu") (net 4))
 (segment (start 164.59 78.7519) (end 166.1495 80.3114) (width 0.5) (layer "F.Cu") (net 8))
 (segment (start 171.4501 79.5019) (end 171.667528 79.5019) (width 0.2) (layer "F.Cu") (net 8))
 (segment (start 174.4732 77.9759) (end 173.4841 77.9759) (width 0.5) (layer "F.Cu") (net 8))
 (segment (start 164.59 77.25) (end 164.59 78.7519) (width 0.5) (layer "F.Cu") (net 8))
 (segment (start 170.6406 80.3114) (end 171.196 79.756) (width 0.5) (layer "F.Cu") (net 8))
 (segment (start 166.1495 80.3114) (end 168.9541 80.3114) (width 0.5) (layer "F.Cu") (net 8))
 (segment (start 172.722648 78.44678) (end 172.93478 78.44678) (width 0.2) (layer "F.Cu") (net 8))
 (segment (start 171.196 79.756) (end 171.4501 79.5019) (width 0.2) (layer "F.Cu") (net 8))
 (segment (start 173.482 77.978) (end 173.40356 77.978) (width 0.5) (layer "F.Cu") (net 8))
 (segment (start 176.2231 76.226) (end 174.4732 77.9759) (width 0.5) (layer "F.Cu") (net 8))
 (segment (start 171.667528 79.5019) (end 172.722648 78.44678) (width 0.2) (layer "F.Cu") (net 8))
 (segment (start 168.9541 80.3114) (end 170.6406 80.3114) (width 0.5) (layer "F.Cu") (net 8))
 (segment (start 173.482 77.978) (end 173.4841 77.9759) (width 0.5) (layer "F.Cu") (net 8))
 (segment (start 176.276 76.226) (end 176.2231 76.226) (width 0.5) (layer "F.Cu") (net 8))
 (segment (start 173.40356 77.978) (end 172.93478 78.44678) (width 0.2) (layer "F.Cu") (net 8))
 (segment (start 157.6219 83.18) (end 162.05 78.7519) (width 0.5) (layer "F.Cu") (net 3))
 (segment (start 157.6219 93.5841) (end 157.6219 83.18) (width 0.5) (layer "F.Cu") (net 3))
 (segment (start 156.718 94.488) (end 157.6219 93.5841) (width 0.5) (layer "F.Cu") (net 3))
 (segment (start 162.05 78.7519) (end 162.05 77.25) (width 0.5) (layer "F.Cu") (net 3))
 (segment (start 160.976 98.044) (end 160.528 98.044) (width 0.5) (layer "F.Cu") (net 1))
 (segment (start 165.86 93.16) (end 160.976 98.044) (width 0.5) (layer "F.Cu") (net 1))
 (segment (start 165.86 91.35) (end 165.86 93.16) (width 0.5) (layer "F.Cu") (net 1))
 (segment (start 158.774 95.988) (end 156.718 98.044) (width 0.5) (layer "F.Cu") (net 2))
 (segment (start 164.59 91.35) (end 164.59 92.547321) (width 0.5) (layer "F.Cu") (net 2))
 (segment (start 161.149321 95.988) (end 158.774 95.988) (width 0.5) (layer "F.Cu") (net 2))
 (segment (start 164.59 92.547321) (end 161.149321 95.988) (width 0.5) (layer "F.Cu") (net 2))
 (segment (start 175.6449 74.676) (end 176.8159 74.676) (width 0.5) (layer "F.Cu") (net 23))
 (segment (start 167.13 77.25) (end 167.13 78.7519) (width 0.5) (layer "F.Cu") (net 23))
 (segment (start 176.8159 74.676) (end 178.071 73.4209) (width 0.5) (layer "F.Cu") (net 23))
 (segment (start 167.13 78.7519) (end 171.569 78.7519) (width 0.5) (layer "F.Cu") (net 23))
 (segment (start 171.569 78.7519) (end 175.6449 74.676) (width 0.5) (layer "F.Cu") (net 23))
 (segment (start 178.071 73.4209) (end 178.071 72.2372) (width 0.5) (layer "F.Cu") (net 23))
 (via (at 178.071 72.2372) (size 0.8) (drill 0.3) (layers "F.Cu" "B.Cu") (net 23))
 (segment (start 178.071 72.2372) (end 177.7877 71.9539) (width 0.5) (layer "B.Cu") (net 23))
 (segment (start 177.7877 71.9539) (end 177.292 71.9539) (width 0.5) (layer "B.Cu") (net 23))
 (segment (start 177.292 70.952) (end 177.292 71.9539) (width 0.5) (layer "B.Cu") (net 23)))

